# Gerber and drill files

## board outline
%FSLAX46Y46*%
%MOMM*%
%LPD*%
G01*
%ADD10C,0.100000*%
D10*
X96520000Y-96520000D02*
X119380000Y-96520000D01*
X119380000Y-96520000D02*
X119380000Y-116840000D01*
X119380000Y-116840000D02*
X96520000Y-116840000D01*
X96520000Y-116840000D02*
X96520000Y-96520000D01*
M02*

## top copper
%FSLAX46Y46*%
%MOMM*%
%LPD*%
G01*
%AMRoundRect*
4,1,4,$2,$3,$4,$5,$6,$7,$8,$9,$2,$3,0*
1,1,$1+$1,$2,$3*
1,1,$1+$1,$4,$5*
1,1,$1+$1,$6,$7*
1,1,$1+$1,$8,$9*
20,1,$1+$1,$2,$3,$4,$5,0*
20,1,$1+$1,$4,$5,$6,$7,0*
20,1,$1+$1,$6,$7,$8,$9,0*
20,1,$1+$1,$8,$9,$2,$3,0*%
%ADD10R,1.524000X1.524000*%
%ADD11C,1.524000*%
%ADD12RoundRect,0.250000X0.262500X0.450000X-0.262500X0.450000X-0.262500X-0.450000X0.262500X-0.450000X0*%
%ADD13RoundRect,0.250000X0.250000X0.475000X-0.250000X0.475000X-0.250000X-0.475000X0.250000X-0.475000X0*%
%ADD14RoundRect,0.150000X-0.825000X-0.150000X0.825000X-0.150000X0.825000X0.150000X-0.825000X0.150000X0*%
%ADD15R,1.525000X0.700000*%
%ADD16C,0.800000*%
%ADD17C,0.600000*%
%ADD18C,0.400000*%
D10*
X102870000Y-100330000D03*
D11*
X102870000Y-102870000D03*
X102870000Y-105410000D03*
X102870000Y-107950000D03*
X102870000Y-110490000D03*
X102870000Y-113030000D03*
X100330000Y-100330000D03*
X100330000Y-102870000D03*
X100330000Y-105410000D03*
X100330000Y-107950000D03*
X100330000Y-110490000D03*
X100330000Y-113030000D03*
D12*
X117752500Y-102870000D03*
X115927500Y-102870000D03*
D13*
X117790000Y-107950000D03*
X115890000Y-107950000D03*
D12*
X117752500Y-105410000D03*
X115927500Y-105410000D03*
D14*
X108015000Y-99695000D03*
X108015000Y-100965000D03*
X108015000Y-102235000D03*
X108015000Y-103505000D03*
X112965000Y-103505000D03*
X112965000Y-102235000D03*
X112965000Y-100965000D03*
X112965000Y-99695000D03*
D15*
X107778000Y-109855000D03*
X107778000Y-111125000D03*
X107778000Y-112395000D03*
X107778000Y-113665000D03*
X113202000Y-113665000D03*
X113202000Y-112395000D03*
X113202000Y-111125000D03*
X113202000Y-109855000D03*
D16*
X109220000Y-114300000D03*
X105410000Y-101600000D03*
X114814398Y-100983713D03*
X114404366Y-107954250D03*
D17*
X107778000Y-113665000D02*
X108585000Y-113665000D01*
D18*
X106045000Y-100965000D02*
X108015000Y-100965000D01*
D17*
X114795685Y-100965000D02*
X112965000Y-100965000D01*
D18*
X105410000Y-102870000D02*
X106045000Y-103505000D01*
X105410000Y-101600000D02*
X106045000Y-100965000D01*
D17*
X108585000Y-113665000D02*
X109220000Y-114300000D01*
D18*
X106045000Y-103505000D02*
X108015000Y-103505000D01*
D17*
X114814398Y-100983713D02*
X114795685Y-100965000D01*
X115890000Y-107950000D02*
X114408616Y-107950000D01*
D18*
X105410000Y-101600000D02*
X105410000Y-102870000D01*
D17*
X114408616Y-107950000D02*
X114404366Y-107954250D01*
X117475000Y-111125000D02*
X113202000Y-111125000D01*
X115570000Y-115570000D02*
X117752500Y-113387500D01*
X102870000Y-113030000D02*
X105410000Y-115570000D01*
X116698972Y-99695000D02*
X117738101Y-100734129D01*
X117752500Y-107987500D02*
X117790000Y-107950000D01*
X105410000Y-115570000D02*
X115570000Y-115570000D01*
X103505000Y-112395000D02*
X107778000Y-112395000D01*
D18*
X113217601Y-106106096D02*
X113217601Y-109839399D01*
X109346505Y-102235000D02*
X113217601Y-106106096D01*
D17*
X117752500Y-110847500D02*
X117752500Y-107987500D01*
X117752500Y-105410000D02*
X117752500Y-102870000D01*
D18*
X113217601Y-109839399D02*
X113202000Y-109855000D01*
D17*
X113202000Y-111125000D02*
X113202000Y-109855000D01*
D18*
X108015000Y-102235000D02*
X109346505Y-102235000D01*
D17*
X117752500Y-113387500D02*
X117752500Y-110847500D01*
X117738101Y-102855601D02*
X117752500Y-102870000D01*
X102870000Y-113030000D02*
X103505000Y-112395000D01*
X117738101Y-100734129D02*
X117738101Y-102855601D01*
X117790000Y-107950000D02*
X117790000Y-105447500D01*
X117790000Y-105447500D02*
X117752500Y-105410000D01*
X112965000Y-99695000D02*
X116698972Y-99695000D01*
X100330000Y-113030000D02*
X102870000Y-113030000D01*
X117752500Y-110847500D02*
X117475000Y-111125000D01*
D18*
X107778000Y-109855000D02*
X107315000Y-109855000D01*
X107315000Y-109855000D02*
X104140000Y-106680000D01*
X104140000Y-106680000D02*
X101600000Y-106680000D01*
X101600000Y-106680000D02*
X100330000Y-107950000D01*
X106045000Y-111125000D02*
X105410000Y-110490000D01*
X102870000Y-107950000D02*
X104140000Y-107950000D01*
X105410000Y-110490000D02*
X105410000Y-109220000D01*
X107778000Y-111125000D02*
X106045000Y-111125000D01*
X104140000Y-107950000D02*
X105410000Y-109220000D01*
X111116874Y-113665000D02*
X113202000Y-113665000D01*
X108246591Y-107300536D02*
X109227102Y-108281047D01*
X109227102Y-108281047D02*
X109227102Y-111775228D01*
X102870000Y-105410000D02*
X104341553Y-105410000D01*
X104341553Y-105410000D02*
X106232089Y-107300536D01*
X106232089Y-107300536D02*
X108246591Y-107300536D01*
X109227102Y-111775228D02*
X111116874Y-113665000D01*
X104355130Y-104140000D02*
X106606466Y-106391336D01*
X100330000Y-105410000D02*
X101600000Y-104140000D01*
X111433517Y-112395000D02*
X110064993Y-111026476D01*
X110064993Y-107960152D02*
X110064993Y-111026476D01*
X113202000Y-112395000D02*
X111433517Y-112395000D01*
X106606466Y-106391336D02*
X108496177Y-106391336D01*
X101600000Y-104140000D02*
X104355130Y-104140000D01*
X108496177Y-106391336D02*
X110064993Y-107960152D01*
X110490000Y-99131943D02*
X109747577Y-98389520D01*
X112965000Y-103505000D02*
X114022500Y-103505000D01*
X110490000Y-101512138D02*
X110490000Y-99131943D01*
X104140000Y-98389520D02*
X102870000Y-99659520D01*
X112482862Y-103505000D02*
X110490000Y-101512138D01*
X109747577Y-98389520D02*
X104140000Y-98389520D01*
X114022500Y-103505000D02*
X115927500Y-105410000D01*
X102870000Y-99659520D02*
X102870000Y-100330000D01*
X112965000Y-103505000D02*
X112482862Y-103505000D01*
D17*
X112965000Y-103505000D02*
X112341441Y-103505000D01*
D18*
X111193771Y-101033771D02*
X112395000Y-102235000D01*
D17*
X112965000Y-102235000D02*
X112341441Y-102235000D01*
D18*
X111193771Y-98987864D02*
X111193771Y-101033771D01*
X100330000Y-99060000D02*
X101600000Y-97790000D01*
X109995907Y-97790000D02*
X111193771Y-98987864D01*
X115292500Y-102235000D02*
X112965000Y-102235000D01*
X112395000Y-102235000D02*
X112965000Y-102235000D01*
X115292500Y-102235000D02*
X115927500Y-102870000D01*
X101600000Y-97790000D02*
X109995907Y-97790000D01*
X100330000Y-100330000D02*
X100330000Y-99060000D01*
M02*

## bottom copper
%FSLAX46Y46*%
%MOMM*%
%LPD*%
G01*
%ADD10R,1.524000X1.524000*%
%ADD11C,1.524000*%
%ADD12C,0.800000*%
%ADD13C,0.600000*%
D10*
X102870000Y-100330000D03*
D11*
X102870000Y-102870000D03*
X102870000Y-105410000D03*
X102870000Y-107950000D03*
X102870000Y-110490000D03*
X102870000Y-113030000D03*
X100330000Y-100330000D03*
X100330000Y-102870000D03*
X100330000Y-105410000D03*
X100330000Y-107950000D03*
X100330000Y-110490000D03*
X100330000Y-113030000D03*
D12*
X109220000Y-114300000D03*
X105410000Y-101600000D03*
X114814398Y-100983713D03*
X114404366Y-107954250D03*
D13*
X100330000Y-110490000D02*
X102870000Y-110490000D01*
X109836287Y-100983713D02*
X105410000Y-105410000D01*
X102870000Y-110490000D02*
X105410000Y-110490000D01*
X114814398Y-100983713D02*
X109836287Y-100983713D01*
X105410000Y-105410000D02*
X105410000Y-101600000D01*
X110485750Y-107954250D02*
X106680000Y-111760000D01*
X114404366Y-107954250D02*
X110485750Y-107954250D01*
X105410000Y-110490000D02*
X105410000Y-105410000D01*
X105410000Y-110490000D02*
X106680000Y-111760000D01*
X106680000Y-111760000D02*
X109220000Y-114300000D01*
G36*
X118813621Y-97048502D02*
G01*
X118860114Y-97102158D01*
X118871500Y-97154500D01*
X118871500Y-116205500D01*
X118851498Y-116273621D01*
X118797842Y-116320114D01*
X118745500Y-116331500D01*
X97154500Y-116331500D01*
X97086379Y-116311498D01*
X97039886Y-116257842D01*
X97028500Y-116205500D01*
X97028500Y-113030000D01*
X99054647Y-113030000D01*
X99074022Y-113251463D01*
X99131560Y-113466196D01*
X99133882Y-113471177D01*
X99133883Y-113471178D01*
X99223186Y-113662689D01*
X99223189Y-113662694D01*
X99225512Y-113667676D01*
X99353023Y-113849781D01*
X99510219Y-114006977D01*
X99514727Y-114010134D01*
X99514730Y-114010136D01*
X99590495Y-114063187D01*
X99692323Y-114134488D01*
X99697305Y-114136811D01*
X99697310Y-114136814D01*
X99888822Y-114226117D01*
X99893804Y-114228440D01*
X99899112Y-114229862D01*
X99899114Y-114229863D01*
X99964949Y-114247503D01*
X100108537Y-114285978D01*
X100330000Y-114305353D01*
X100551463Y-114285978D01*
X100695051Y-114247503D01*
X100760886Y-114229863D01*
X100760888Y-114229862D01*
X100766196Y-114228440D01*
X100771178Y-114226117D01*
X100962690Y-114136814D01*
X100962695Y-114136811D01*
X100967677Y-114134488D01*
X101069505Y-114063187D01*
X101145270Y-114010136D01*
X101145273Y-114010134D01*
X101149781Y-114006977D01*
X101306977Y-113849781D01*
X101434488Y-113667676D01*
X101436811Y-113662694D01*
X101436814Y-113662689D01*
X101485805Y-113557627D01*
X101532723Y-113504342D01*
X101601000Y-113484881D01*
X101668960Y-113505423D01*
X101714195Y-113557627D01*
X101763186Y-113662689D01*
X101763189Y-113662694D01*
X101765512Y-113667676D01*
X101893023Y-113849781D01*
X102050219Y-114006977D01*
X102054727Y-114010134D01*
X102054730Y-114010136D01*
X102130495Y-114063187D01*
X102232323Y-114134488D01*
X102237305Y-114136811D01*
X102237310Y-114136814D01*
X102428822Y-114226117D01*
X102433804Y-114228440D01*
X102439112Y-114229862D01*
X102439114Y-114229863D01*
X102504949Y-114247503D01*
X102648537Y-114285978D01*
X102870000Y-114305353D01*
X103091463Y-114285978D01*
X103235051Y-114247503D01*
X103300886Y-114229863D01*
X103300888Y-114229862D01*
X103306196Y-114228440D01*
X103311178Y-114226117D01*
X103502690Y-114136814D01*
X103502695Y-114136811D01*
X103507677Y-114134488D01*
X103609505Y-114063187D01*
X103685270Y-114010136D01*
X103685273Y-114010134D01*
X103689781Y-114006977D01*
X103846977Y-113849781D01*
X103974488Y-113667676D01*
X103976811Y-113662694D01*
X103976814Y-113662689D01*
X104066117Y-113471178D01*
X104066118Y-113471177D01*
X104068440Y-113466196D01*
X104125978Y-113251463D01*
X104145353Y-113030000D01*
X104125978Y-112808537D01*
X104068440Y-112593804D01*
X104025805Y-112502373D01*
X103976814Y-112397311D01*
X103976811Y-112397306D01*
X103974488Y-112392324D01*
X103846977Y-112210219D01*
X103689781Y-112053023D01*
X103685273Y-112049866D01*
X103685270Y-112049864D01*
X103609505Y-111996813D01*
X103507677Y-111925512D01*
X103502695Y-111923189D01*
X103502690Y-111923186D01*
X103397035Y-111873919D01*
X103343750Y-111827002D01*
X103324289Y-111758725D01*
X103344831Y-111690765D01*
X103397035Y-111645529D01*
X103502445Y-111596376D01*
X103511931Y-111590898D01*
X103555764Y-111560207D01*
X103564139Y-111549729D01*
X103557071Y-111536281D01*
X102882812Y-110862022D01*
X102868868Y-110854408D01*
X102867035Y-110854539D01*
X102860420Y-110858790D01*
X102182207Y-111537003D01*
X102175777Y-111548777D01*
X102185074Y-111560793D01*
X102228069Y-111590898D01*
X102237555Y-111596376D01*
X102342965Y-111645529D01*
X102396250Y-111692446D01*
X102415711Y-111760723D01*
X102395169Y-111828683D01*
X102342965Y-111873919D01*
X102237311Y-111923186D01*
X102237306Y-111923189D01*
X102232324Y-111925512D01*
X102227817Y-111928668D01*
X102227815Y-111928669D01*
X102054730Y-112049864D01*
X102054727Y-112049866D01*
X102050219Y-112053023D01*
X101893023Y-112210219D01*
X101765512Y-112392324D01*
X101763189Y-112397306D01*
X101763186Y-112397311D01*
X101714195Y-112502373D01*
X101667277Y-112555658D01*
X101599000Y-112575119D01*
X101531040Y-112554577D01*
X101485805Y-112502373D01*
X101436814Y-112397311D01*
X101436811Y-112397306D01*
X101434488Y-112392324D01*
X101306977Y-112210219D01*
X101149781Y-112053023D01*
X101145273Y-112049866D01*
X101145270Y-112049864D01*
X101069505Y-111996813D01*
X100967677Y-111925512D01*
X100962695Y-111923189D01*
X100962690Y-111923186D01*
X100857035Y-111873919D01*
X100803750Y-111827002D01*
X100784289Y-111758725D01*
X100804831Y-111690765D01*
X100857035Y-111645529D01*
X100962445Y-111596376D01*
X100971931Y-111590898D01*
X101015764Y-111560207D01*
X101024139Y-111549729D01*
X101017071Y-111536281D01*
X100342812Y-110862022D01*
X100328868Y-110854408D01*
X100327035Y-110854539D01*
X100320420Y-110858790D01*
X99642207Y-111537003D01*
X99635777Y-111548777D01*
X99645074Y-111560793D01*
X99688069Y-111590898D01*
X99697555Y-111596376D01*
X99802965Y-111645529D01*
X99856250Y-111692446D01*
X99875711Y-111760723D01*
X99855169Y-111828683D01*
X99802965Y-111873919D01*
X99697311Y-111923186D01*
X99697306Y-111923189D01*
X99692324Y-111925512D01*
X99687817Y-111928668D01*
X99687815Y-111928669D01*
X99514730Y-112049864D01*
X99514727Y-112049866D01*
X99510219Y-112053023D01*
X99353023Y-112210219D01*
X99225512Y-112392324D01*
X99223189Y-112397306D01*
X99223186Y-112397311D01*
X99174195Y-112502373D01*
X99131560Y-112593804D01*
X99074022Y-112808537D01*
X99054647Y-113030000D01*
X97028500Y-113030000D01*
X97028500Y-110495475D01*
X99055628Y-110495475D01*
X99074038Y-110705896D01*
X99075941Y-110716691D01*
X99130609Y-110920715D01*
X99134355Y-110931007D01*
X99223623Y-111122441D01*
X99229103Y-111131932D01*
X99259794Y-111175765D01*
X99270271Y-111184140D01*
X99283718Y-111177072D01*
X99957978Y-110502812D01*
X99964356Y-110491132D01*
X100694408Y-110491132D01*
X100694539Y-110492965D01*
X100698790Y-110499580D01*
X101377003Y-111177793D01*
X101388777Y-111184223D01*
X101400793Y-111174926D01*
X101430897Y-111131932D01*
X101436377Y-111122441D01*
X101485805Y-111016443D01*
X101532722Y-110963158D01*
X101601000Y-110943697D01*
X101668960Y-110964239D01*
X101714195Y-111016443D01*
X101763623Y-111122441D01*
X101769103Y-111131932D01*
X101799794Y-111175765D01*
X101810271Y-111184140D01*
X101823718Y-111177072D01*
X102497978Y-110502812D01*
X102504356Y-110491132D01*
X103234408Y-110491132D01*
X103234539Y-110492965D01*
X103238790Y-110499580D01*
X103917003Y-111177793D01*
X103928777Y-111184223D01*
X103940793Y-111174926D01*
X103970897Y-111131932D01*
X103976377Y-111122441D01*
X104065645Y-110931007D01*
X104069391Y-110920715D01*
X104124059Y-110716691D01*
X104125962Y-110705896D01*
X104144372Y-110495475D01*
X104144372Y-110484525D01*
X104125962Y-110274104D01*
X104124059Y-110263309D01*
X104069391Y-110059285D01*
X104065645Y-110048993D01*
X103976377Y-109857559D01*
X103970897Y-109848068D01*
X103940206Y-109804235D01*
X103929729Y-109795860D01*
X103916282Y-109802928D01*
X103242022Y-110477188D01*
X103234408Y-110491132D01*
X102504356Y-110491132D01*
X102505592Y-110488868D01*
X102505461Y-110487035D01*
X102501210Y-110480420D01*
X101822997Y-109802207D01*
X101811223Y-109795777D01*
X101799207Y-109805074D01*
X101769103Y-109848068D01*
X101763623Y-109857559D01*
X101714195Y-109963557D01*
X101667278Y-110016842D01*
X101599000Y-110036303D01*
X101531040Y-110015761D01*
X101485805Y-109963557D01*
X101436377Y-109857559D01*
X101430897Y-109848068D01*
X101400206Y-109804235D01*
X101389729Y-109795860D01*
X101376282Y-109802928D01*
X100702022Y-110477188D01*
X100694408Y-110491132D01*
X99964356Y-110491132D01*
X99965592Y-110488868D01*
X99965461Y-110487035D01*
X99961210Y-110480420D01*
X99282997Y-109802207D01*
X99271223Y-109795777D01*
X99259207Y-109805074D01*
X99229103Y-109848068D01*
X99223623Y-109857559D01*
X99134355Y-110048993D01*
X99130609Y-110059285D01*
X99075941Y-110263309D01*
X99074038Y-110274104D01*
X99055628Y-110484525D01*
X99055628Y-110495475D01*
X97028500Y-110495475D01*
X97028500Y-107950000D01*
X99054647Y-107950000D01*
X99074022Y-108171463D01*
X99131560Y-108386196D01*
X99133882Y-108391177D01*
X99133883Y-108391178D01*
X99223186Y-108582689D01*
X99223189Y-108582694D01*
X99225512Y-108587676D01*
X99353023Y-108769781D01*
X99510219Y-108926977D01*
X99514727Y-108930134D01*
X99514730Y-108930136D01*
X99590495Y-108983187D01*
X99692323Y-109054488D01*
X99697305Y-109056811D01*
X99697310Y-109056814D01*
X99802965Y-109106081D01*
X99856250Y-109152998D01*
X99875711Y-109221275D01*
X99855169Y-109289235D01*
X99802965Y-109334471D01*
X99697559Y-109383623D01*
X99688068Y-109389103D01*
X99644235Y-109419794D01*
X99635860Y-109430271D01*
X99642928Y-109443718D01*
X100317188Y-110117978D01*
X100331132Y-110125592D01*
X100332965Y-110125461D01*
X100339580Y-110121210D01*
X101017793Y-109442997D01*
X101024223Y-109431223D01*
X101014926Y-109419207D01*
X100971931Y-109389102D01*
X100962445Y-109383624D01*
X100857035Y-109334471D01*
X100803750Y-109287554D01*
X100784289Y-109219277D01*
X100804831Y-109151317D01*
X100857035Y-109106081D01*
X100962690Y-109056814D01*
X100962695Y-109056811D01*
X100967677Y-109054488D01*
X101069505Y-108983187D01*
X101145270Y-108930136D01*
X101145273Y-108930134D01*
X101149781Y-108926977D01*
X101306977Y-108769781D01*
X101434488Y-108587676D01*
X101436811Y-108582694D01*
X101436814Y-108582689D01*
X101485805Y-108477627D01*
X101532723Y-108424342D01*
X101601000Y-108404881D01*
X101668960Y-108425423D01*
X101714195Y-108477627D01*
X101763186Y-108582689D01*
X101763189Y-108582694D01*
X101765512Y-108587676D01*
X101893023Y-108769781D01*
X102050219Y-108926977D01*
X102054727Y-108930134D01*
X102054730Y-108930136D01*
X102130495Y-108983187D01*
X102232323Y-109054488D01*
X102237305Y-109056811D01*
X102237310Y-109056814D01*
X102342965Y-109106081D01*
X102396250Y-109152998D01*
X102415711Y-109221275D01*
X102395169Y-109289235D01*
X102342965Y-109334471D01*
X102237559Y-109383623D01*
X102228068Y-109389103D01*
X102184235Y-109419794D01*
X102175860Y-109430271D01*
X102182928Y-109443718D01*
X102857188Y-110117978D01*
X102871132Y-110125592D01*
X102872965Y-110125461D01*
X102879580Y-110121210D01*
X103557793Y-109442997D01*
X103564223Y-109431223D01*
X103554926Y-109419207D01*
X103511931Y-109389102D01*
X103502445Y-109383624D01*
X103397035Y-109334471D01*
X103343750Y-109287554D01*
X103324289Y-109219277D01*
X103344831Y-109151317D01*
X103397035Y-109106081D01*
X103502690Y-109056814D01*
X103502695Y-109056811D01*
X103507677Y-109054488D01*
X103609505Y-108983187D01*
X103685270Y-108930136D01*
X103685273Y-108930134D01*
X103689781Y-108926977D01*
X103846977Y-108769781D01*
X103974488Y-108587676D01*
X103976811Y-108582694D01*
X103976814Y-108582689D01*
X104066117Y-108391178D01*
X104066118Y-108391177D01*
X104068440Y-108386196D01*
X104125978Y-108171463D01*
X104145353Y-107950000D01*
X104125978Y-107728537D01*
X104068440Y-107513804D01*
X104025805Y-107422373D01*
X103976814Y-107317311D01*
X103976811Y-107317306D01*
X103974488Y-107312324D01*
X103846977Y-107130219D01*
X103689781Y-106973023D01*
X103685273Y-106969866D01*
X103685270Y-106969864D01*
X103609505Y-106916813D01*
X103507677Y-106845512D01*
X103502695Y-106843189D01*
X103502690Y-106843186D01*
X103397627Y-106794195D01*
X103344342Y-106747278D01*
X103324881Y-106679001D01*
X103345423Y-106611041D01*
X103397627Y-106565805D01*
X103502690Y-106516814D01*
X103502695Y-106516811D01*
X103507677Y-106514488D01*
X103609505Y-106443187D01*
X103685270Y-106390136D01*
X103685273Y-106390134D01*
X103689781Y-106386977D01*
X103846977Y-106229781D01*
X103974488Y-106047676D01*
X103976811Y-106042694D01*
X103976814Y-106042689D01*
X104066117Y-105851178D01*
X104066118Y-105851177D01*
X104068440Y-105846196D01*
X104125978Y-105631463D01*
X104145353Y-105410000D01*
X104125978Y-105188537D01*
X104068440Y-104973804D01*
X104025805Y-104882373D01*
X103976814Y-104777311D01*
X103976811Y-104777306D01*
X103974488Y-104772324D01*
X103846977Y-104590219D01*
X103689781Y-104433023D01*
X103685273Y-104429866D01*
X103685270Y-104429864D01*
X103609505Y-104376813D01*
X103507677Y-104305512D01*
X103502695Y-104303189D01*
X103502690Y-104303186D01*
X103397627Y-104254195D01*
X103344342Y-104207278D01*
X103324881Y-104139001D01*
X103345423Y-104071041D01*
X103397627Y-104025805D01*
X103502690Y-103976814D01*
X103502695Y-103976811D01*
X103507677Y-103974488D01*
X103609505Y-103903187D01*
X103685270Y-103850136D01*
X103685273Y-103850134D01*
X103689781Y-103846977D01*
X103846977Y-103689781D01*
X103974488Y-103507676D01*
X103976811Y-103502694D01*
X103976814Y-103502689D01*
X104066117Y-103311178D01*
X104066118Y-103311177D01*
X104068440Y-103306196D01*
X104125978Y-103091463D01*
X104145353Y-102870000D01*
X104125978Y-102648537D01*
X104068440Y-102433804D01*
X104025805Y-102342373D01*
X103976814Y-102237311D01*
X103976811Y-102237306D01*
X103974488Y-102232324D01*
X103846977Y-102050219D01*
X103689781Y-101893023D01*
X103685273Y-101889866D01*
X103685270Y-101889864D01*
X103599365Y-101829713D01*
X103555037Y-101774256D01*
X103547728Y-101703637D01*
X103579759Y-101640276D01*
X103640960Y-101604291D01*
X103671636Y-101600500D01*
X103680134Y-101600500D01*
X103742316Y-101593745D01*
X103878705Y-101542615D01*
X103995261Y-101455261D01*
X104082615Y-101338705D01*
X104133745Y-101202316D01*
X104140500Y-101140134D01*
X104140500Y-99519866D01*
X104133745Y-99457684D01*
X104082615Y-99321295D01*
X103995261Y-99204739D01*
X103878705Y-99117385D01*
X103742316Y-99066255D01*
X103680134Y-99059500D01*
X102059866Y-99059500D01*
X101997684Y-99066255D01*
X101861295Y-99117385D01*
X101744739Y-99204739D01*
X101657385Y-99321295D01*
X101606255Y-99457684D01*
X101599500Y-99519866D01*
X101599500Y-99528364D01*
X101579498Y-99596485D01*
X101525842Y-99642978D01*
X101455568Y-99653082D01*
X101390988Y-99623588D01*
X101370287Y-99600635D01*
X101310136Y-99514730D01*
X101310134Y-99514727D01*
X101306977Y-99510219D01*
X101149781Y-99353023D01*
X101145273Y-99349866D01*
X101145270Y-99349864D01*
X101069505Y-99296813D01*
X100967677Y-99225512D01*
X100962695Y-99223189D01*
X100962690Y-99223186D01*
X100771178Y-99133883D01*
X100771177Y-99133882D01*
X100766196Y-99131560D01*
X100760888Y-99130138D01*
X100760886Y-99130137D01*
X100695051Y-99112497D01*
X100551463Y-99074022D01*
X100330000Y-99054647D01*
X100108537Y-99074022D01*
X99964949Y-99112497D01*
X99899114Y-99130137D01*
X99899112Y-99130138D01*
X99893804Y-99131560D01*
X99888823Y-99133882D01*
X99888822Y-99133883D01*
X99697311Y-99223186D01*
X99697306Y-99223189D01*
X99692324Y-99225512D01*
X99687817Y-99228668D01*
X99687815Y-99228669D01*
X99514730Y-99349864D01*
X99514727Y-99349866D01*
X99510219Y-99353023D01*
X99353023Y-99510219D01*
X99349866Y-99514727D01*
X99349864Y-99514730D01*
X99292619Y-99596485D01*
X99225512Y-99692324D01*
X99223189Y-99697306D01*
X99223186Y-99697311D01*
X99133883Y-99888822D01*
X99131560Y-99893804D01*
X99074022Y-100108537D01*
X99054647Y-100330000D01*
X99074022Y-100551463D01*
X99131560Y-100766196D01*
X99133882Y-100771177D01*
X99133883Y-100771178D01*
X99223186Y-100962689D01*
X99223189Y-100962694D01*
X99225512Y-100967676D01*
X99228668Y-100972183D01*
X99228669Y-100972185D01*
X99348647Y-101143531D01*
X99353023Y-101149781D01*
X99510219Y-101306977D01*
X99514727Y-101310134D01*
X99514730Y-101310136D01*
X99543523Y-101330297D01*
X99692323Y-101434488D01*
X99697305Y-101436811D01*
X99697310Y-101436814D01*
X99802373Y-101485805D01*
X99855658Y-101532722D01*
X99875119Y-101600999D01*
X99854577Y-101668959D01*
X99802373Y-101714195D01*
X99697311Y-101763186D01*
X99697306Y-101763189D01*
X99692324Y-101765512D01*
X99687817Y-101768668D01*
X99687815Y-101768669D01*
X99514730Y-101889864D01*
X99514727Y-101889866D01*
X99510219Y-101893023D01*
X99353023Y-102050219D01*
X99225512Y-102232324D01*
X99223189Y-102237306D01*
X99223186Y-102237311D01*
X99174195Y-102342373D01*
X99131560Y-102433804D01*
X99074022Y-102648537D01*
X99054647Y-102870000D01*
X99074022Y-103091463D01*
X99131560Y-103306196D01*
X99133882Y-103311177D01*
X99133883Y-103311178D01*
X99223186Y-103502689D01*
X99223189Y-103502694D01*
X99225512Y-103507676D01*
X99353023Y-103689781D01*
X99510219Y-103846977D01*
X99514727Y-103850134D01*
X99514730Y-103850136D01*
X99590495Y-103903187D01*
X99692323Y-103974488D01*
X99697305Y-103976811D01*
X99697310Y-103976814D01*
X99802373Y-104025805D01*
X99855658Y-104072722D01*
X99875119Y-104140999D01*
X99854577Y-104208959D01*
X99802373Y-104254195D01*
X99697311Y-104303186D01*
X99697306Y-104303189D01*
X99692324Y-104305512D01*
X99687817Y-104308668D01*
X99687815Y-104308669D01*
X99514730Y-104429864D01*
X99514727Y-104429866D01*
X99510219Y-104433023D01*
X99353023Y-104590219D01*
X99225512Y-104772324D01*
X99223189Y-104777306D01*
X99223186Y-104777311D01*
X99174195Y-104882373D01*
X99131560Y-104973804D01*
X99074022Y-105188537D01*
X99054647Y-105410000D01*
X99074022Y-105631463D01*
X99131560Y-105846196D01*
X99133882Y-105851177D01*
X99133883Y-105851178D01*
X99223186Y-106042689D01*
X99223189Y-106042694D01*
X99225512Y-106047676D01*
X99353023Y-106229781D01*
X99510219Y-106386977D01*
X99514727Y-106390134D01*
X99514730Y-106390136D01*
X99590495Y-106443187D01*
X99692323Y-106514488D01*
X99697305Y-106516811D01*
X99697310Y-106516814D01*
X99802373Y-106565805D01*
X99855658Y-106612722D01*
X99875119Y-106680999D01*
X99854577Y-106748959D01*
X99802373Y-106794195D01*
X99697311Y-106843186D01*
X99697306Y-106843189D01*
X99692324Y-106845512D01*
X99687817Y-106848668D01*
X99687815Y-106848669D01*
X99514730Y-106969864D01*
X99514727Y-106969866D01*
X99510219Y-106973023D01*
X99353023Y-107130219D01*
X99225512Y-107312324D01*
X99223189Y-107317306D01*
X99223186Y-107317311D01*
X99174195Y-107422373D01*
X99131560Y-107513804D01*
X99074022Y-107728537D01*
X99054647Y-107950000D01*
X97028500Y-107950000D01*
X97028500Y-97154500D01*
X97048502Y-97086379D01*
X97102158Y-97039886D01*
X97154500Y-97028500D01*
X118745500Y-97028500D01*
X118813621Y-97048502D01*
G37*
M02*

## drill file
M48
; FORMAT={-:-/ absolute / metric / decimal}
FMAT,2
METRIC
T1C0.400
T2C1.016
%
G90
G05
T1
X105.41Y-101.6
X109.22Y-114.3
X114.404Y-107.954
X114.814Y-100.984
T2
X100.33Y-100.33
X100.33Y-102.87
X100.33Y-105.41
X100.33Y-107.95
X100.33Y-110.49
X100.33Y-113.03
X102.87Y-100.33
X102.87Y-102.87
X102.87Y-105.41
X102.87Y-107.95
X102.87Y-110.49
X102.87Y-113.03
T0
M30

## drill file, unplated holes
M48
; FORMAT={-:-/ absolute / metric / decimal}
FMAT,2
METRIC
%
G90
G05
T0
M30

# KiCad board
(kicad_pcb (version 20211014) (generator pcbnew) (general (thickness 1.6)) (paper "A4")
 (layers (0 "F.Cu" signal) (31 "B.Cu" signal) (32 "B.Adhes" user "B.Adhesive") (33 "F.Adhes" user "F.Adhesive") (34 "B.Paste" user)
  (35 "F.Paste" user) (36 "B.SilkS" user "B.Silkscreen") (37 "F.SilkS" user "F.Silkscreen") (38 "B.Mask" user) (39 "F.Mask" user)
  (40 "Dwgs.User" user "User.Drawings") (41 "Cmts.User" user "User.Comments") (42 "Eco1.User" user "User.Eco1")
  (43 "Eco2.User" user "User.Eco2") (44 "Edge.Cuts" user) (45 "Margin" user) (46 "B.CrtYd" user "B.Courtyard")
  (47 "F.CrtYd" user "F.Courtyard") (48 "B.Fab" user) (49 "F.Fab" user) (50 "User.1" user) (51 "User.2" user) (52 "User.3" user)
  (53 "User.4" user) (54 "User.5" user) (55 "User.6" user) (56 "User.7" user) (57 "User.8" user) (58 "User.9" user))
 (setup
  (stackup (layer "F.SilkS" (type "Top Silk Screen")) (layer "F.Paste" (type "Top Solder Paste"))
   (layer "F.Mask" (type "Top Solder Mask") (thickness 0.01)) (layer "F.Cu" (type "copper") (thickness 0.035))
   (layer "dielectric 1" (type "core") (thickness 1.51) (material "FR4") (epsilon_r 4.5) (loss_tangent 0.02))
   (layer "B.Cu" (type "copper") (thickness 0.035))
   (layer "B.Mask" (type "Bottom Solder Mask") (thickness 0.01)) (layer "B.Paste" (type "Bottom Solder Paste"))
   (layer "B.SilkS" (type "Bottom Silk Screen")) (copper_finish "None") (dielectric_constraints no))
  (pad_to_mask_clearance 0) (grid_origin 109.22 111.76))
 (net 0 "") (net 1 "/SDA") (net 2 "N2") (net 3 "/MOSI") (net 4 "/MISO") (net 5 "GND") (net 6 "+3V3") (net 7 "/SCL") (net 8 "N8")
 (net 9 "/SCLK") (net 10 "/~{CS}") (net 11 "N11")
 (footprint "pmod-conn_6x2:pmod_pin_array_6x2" (layer "F.Cu") (at 101.6 106.68)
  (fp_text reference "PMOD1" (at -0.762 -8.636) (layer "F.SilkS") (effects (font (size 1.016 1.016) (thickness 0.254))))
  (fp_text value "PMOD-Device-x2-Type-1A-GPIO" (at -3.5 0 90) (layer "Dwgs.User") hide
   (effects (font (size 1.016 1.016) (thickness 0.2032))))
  (pad "1" thru_hole rect locked (at 1.27 -6.35) (size 1.524 1.524) (drill 1.016) (layers *.Cu *.Mask "F.SilkS") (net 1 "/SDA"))
  (pad "2" thru_hole circle locked (at 1.27 -3.81 270) (size 1.524 1.524) (drill 1.016) (layers *.Cu *.Mask "F.SilkS") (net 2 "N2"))
  (pad "3" thru_hole circle locked (at 1.27 -1.27 270) (size 1.524 1.524) (drill 1.016) (layers *.Cu *.Mask "F.SilkS") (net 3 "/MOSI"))
  (pad "4" thru_hole circle locked (at 1.27 1.27 270) (size 1.524 1.524) (drill 1.016) (layers *.Cu *.Mask "F.SilkS") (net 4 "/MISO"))
  (pad "5" thru_hole circle locked (at 1.27 3.81 270) (size 1.524 1.524) (drill 1.016) (layers *.Cu *.Mask "F.SilkS") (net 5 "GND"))
  (pad "6" thru_hole circle locked (at 1.27 6.35 270) (size 1.524 1.524) (drill 1.016) (layers *.Cu *.Mask "F.SilkS") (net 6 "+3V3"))
  (pad "7" thru_hole circle locked (at -1.27 -6.35 270) (size 1.524 1.524) (drill 1.016) (layers *.Cu *.Mask "F.SilkS") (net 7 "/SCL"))
  (pad "8" thru_hole circle locked (at -1.27 -3.81 270) (size 1.524 1.524) (drill 1.016) (layers *.Cu *.Mask "F.SilkS") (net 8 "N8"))
  (pad "9" thru_hole circle locked (at -1.27 -1.27 270) (size 1.524 1.524) (drill 1.016) (layers *.Cu *.Mask "F.SilkS") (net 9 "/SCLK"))
  (pad "10" thru_hole circle locked (at -1.27 1.27 270) (size 1.524 1.524) (drill 1.016) (layers *.Cu *.Mask "F.SilkS") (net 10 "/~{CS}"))
  (pad "11" thru_hole circle locked (at -1.27 3.81 270) (size 1.524 1.524) (drill 1.016) (layers *.Cu *.Mask "F.SilkS") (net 5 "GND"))
  (pad "12" thru_hole circle locked (at -1.27 6.35 270) (size 1.524 1.524) (drill 1.016) (layers *.Cu *.Mask "F.SilkS") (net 6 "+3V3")))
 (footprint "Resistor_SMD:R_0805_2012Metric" (layer "F.Cu") (at 116.84 102.87 180)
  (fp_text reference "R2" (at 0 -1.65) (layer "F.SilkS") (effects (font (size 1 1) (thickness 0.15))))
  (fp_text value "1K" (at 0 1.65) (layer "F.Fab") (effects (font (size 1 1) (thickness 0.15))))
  (pad "1" smd roundrect (at -0.9125 0 180) (size 1.025 1.4) (layers "F.Cu" "F.Paste" "F.Mask") (roundrect_rratio 0.243902439)
   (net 6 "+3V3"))
  (pad "2" smd roundrect (at 0.9125 0 180) (size 1.025 1.4) (layers "F.Cu" "F.Paste" "F.Mask") (roundrect_rratio 0.243902439) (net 7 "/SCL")))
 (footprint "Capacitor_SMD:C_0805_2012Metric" (layer "F.Cu") (at 116.84 107.95 180)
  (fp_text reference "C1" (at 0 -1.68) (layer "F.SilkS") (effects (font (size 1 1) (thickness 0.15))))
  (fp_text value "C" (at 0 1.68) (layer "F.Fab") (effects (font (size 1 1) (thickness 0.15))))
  (pad "1" smd roundrect (at -0.95 0 180) (size 1 1.45) (layers "F.Cu" "F.Paste" "F.Mask") (roundrect_rratio 0.25) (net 6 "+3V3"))
  (pad "2" smd roundrect (at 0.95 0 180) (size 1 1.45) (layers "F.Cu" "F.Paste" "F.Mask") (roundrect_rratio 0.25) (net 5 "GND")))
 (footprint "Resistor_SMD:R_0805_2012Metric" (layer "F.Cu") (at 116.84 105.41 180)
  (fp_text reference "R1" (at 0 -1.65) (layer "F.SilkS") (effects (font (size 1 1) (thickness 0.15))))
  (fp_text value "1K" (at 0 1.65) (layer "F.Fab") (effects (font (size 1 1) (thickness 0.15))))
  (pad "1" smd roundrect (at -0.9125 0 180) (size 1.025 1.4) (layers "F.Cu" "F.Paste" "F.Mask") (roundrect_rratio 0.243902439)
   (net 6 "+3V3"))
  (pad "2" smd roundrect (at 0.9125 0 180) (size 1.025 1.4) (layers "F.Cu" "F.Paste" "F.Mask") (roundrect_rratio 0.243902439) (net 1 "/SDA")))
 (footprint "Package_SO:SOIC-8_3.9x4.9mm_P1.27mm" (layer "F.Cu") (at 110.49 101.6)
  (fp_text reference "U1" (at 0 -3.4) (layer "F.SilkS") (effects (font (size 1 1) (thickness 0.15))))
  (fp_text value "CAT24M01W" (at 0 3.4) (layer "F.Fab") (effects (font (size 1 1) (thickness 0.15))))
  (pad "1" smd roundrect (at -2.475 -1.905) (size 1.95 0.6) (layers "F.Cu" "F.Paste" "F.Mask") (roundrect_rratio 0.25) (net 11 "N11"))
  (pad "2" smd roundrect (at -2.475 -0.635) (size 1.95 0.6) (layers "F.Cu" "F.Paste" "F.Mask") (roundrect_rratio 0.25) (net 5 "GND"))
  (pad "3" smd roundrect (at -2.475 0.635) (size 1.95 0.6) (layers "F.Cu" "F.Paste" "F.Mask") (roundrect_rratio 0.25) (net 6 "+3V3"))
  (pad "4" smd roundrect (at -2.475 1.905) (size 1.95 0.6) (layers "F.Cu" "F.Paste" "F.Mask") (roundrect_rratio 0.25) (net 5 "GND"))
  (pad "5" smd roundrect (at 2.475 1.905) (size 1.95 0.6) (layers "F.Cu" "F.Paste" "F.Mask") (roundrect_rratio 0.25) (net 1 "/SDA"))
  (pad "6" smd roundrect (at 2.475 0.635) (size 1.95 0.6) (layers "F.Cu" "F.Paste" "F.Mask") (roundrect_rratio 0.25) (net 7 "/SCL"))
  (pad "7" smd roundrect (at 2.475 -0.635) (size 1.95 0.6) (layers "F.Cu" "F.Paste" "F.Mask") (roundrect_rratio 0.25) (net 5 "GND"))
  (pad "8" smd roundrect (at 2.475 -1.905) (size 1.95 0.6) (layers "F.Cu" "F.Paste" "F.Mask") (roundrect_rratio 0.25) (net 6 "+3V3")))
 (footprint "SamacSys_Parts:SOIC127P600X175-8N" (layer "F.Cu") (at 110.49 111.76)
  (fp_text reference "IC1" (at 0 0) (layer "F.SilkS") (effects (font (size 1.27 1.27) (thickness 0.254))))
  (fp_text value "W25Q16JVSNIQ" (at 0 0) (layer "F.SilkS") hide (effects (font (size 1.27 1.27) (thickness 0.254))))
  (pad "1" smd rect (at -2.712 -1.905 90) (size 0.7 1.525) (layers "F.Cu" "F.Paste" "F.Mask") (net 10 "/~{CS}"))
  (pad "2" smd rect (at -2.712 -0.635 90) (size 0.7 1.525) (layers "F.Cu" "F.Paste" "F.Mask") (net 4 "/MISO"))
  (pad "3" smd rect (at -2.712 0.635 90) (size 0.7 1.525) (layers "F.Cu" "F.Paste" "F.Mask") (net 6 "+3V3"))
  (pad "4" smd rect (at -2.712 1.905 90) (size 0.7 1.525) (layers "F.Cu" "F.Paste" "F.Mask") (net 5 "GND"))
  (pad "5" smd rect (at 2.712 1.905 90) (size 0.7 1.525) (layers "F.Cu" "F.Paste" "F.Mask") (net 3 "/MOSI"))
  (pad "6" smd rect (at 2.712 0.635 90) (size 0.7 1.525) (layers "F.Cu" "F.Paste" "F.Mask") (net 9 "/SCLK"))
  (pad "7" smd rect (at 2.712 -0.635 90) (size 0.7 1.525) (layers "F.Cu" "F.Paste" "F.Mask") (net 6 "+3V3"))
  (pad "8" smd rect (at 2.712 -1.905 90) (size 0.7 1.525) (layers "F.Cu" "F.Paste" "F.Mask") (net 6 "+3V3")))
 (gr_rect (start 96.52 96.52) (end 119.38 116.84) (layer "Edge.Cuts") (width 0.1) (fill none))
 (segment (start 107.778 113.665) (end 108.585 113.665) (width 0.6) (layer "F.Cu") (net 5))
 (segment (start 106.045 100.965) (end 108.015 100.965) (width 0.4) (layer "F.Cu") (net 5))
 (segment (start 114.795685 100.965) (end 112.965 100.965) (width 0.6) (layer "F.Cu") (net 5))
 (segment (start 105.41 102.87) (end 106.045 103.505) (width 0.4) (layer "F.Cu") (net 5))
 (segment (start 105.41 101.6) (end 106.045 100.965) (width 0.4) (layer "F.Cu") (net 5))
 (segment (start 108.585 113.665) (end 109.22 114.3) (width 0.6) (layer "F.Cu") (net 5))
 (segment (start 106.045 103.505) (end 108.015 103.505) (width 0.4) (layer "F.Cu") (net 5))
 (segment (start 114.814398 100.983713) (end 114.795685 100.965) (width 0.6) (layer "F.Cu") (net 5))
 (segment (start 115.89 107.95) (end 114.408616 107.95) (width 0.6) (layer "F.Cu") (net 5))
 (segment (start 105.41 101.6) (end 105.41 102.87) (width 0.4) (layer "F.Cu") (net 5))
 (segment (start 114.408616 107.95) (end 114.404366 107.95425) (width 0.6) (layer "F.Cu") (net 5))
 (via (at 109.22 114.3) (size 0.8) (drill 0.4) (layers "F.Cu" "B.Cu") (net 5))
 (via (at 105.41 101.6) (size 0.8) (drill 0.4) (layers "F.Cu" "B.Cu") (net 5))
 (via (at 114.814398 100.983713) (size 0.8) (drill 0.4) (layers "F.Cu" "B.Cu") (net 5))
 (via (at 114.404366 107.95425) (size 0.8) (drill 0.4) (layers "F.Cu" "B.Cu") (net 5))
 (segment (start 100.33 110.49) (end 102.87 110.49) (width 0.6) (layer "B.Cu") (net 5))
 (segment (start 109.836287 100.983713) (end 105.41 105.41) (width 0.6) (layer "B.Cu") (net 5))
 (segment (start 102.87 110.49) (end 105.41 110.49) (width 0.6) (layer "B.Cu") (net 5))
 (segment (start 114.814398 100.983713) (end 109.836287 100.983713) (width 0.6) (layer "B.Cu") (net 5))
 (segment (start 105.41 105.41) (end 105.41 101.6) (width 0.6) (layer "B.Cu") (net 5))
 (segment (start 110.48575 107.95425) (end 106.68 111.76) (width 0.6) (layer "B.Cu") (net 5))
 (segment (start 114.404366 107.95425) (end 110.48575 107.95425) (width 0.6) (layer "B.Cu") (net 5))
 (segment (start 105.41 110.49) (end 105.41 105.41) (width 0.6) (layer "B.Cu") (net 5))
 (segment (start 105.41 110.49) (end 106.68 111.76) (width 0.6) (layer "B.Cu") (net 5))
 (segment (start 106.68 111.76) (end 109.22 114.3) (width 0.6) (layer "B.Cu") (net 5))
 (segment (start 117.475 111.125) (end 113.202 111.125) (width 0.6) (layer "F.Cu") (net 6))
 (segment (start 115.57 115.57) (end 117.7525 113.3875) (width 0.6) (layer "F.Cu") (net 6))
 (segment (start 102.87 113.03) (end 105.41 115.57) (width 0.6) (layer "F.Cu") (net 6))
 (segment (start 116.698972 99.695) (end 117.738101 100.734129) (width 0.6) (layer "F.Cu") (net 6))
 (segment (start 117.7525 107.9875) (end 117.79 107.95) (width 0.6) (layer "F.Cu") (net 6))
 (segment (start 105.41 115.57) (end 115.57 115.57) (width 0.6) (layer "F.Cu") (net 6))
 (segment (start 103.505 112.395) (end 107.778 112.395) (width 0.6) (layer "F.Cu") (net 6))
 (segment (start 113.217601 106.106096) (end 113.217601 109.839399) (width 0.4) (layer "F.Cu") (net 6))
 (segment (start 109.346505 102.235) (end 113.217601 106.106096) (width 0.4) (layer "F.Cu") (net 6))
 (segment (start 117.7525 110.8475) (end 117.7525 107.9875) (width 0.6) (layer "F.Cu") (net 6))
 (segment (start 117.7525 105.41) (end 117.7525 102.87) (width 0.6) (layer "F.Cu") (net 6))
 (segment (start 113.217601 109.839399) (end 113.202 109.855) (width 0.4) (layer "F.Cu") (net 6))
 (segment (start 113.202 111.125) (end 113.202 109.855) (width 0.6) (layer "F.Cu") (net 6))
 (segment (start 108.015 102.235) (end 109.346505 102.235) (width 0.4) (layer "F.Cu") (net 6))
 (segment (start 117.7525 113.3875) (end 117.7525 110.8475) (width 0.6) (layer "F.Cu") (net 6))
 (segment (start 117.738101 102.855601) (end 117.7525 102.87) (width 0.6) (layer "F.Cu") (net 6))
 (segment (start 102.87 113.03) (end 103.505 112.395) (width 0.6) (layer "F.Cu") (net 6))
 (segment (start 117.738101 100.734129) (end 117.738101 102.855601) (width 0.6) (layer "F.Cu") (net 6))
 (segment (start 117.79 107.95) (end 117.79 105.4475) (width 0.6) (layer "F.Cu") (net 6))
 (segment (start 117.79 105.4475) (end 117.7525 105.41) (width 0.6) (layer "F.Cu") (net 6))
 (segment (start 112.965 99.695) (end 116.698972 99.695) (width 0.6) (layer "F.Cu") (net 6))
 (segment (start 100.33 113.03) (end 102.87 113.03) (width 0.6) (layer "F.Cu") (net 6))
 (segment (start 117.7525 110.8475) (end 117.475 111.125) (width 0.6) (layer "F.Cu") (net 6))
 (segment (start 107.778 109.855) (end 107.315 109.855) (width 0.4) (layer "F.Cu") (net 10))
 (segment (start 107.315 109.855) (end 104.14 106.68) (width 0.4) (layer "F.Cu") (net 10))
 (segment (start 104.14 106.68) (end 101.6 106.68) (width 0.4) (layer "F.Cu") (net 10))
 (segment (start 101.6 106.68) (end 100.33 107.95) (width 0.4) (layer "F.Cu") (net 10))
 (segment (start 106.045 111.125) (end 105.41 110.49) (width 0.4) (layer "F.Cu") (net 4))
 (segment (start 102.87 107.95) (end 104.14 107.95) (width 0.4) (layer "F.Cu") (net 4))
 (segment (start 105.41 110.49) (end 105.41 109.22) (width 0.4) (layer "F.Cu") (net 4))
 (segment (start 107.778 111.125) (end 106.045 111.125) (width 0.4) (layer "F.Cu") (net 4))
 (segment (start 104.14 107.95) (end 105.41 109.22) (width 0.4) (layer "F.Cu") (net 4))
 (segment (start 111.116874 113.665) (end 113.202 113.665) (width 0.4) (layer "F.Cu") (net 3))
 (segment (start 108.246591 107.300536) (end 109.227102 108.281047) (width 0.4) (layer "F.Cu") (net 3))
 (segment (start 109.227102 108.281047) (end 109.227102 111.775228) (width 0.4) (layer "F.Cu") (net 3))
 (segment (start 102.87 105.41) (end 104.341553 105.41) (width 0.4) (layer "F.Cu") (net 3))
 (segment (start 104.341553 105.41) (end 106.232089 107.300536) (width 0.4) (layer "F.Cu") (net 3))
 (segment (start 106.232089 107.300536) (end 108.246591 107.300536) (width 0.4) (layer "F.Cu") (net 3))
 (segment (start 109.227102 111.775228) (end 111.116874 113.665) (width 0.4) (layer "F.Cu") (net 3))
 (segment (start 104.35513 104.14) (end 106.606466 106.391336) (width 0.4) (layer "F.Cu") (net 9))
 (segment (start 100.33 105.41) (end 101.6 104.14) (width 0.4) (layer "F.Cu") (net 9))
 (segment (start 111.433517 112.395) (end 110.064993 111.026476) (width 0.4) (layer "F.Cu") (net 9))
 (segment (start 110.064993 107.960152) (end 110.064993 111.026476) (width 0.4) (layer "F.Cu") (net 9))
 (segment (start 113.202 112.395) (end 111.433517 112.395) (width 0.4) (layer "F.Cu") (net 9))
 (segment (start 106.606466 106.391336) (end 108.496177 106.391336) (width 0.4) (layer "F.Cu") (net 9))
 (segment (start 101.6 104.14) (end 104.35513 104.14) (width 0.4) (layer "F.Cu") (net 9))
 (segment (start 108.496177 106.391336) (end 110.064993 107.960152) (width 0.4) (layer "F.Cu") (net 9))
 (segment (start 110.49 99.131943) (end 109.747577 98.38952) (width 0.4) (layer "F.Cu") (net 1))
 (segment (start 112.965 103.505) (end 114.0225 103.505) (width 0.4) (layer "F.Cu") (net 1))
 (segment (start 110.49 101.512138) (end 110.49 99.131943) (width 0.4) (layer "F.Cu") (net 1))
 (segment (start 104.14 98.38952) (end 102.87 99.65952) (width 0.4) (layer "F.Cu") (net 1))
 (segment (start 112.482862 103.505) (end 110.49 101.512138) (width 0.4) (layer "F.Cu") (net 1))
 (segment (start 109.747577 98.38952) (end 104.14 98.38952) (width 0.4) (layer "F.Cu") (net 1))
 (segment (start 114.0225 103.505) (end 115.9275 105.41) (width 0.4) (layer "F.Cu") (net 1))
 (segment (start 102.87 99.65952) (end 102.87 100.33) (width 0.4) (layer "F.Cu") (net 1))
 (segment (start 112.965 103.505) (end 112.482862 103.505) (width 0.4) (layer "F.Cu") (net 1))
 (segment (start 112.965 103.505) (end 112.341441 103.505) (width 0.6) (layer "F.Cu") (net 1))
 (segment (start 111.193771 101.033771) (end 112.395 102.235) (width 0.4) (layer "F.Cu") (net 7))
 (segment (start 112.965 102.235) (end 112.341441 102.235) (width 0.6) (layer "F.Cu") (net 7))
 (segment (start 111.193771 98.987864) (end 111.193771 101.033771) (width 0.4) (layer "F.Cu") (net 7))
 (segment (start 100.33 99.06) (end 101.6 97.79) (width 0.4) (layer "F.Cu") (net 7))
 (segment (start 109.995907 97.79) (end 111.193771 98.987864) (width 0.4) (layer "F.Cu") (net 7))
 (segment (start 115.2925 102.235) (end 112.965 102.235) (width 0.4) (layer "F.Cu") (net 7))
 (segment (start 112.395 102.235) (end 112.965 102.235) (width 0.4) (layer "F.Cu") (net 7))
 (segment (start 115.2925 102.235) (end 115.9275 102.87) (width 0.4) (layer "F.Cu") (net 7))
 (segment (start 101.6 97.79) (end 109.995907 97.79) (width 0.4) (layer "F.Cu") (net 7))
 (segment (start 100.33 100.33) (end 100.33 99.06) (width 0.4) (layer "F.Cu") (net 7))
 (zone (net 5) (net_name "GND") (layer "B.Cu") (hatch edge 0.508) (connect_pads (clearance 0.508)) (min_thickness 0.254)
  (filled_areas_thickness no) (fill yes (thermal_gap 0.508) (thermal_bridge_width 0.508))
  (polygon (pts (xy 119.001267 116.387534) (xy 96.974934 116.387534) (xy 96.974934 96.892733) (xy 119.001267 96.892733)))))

